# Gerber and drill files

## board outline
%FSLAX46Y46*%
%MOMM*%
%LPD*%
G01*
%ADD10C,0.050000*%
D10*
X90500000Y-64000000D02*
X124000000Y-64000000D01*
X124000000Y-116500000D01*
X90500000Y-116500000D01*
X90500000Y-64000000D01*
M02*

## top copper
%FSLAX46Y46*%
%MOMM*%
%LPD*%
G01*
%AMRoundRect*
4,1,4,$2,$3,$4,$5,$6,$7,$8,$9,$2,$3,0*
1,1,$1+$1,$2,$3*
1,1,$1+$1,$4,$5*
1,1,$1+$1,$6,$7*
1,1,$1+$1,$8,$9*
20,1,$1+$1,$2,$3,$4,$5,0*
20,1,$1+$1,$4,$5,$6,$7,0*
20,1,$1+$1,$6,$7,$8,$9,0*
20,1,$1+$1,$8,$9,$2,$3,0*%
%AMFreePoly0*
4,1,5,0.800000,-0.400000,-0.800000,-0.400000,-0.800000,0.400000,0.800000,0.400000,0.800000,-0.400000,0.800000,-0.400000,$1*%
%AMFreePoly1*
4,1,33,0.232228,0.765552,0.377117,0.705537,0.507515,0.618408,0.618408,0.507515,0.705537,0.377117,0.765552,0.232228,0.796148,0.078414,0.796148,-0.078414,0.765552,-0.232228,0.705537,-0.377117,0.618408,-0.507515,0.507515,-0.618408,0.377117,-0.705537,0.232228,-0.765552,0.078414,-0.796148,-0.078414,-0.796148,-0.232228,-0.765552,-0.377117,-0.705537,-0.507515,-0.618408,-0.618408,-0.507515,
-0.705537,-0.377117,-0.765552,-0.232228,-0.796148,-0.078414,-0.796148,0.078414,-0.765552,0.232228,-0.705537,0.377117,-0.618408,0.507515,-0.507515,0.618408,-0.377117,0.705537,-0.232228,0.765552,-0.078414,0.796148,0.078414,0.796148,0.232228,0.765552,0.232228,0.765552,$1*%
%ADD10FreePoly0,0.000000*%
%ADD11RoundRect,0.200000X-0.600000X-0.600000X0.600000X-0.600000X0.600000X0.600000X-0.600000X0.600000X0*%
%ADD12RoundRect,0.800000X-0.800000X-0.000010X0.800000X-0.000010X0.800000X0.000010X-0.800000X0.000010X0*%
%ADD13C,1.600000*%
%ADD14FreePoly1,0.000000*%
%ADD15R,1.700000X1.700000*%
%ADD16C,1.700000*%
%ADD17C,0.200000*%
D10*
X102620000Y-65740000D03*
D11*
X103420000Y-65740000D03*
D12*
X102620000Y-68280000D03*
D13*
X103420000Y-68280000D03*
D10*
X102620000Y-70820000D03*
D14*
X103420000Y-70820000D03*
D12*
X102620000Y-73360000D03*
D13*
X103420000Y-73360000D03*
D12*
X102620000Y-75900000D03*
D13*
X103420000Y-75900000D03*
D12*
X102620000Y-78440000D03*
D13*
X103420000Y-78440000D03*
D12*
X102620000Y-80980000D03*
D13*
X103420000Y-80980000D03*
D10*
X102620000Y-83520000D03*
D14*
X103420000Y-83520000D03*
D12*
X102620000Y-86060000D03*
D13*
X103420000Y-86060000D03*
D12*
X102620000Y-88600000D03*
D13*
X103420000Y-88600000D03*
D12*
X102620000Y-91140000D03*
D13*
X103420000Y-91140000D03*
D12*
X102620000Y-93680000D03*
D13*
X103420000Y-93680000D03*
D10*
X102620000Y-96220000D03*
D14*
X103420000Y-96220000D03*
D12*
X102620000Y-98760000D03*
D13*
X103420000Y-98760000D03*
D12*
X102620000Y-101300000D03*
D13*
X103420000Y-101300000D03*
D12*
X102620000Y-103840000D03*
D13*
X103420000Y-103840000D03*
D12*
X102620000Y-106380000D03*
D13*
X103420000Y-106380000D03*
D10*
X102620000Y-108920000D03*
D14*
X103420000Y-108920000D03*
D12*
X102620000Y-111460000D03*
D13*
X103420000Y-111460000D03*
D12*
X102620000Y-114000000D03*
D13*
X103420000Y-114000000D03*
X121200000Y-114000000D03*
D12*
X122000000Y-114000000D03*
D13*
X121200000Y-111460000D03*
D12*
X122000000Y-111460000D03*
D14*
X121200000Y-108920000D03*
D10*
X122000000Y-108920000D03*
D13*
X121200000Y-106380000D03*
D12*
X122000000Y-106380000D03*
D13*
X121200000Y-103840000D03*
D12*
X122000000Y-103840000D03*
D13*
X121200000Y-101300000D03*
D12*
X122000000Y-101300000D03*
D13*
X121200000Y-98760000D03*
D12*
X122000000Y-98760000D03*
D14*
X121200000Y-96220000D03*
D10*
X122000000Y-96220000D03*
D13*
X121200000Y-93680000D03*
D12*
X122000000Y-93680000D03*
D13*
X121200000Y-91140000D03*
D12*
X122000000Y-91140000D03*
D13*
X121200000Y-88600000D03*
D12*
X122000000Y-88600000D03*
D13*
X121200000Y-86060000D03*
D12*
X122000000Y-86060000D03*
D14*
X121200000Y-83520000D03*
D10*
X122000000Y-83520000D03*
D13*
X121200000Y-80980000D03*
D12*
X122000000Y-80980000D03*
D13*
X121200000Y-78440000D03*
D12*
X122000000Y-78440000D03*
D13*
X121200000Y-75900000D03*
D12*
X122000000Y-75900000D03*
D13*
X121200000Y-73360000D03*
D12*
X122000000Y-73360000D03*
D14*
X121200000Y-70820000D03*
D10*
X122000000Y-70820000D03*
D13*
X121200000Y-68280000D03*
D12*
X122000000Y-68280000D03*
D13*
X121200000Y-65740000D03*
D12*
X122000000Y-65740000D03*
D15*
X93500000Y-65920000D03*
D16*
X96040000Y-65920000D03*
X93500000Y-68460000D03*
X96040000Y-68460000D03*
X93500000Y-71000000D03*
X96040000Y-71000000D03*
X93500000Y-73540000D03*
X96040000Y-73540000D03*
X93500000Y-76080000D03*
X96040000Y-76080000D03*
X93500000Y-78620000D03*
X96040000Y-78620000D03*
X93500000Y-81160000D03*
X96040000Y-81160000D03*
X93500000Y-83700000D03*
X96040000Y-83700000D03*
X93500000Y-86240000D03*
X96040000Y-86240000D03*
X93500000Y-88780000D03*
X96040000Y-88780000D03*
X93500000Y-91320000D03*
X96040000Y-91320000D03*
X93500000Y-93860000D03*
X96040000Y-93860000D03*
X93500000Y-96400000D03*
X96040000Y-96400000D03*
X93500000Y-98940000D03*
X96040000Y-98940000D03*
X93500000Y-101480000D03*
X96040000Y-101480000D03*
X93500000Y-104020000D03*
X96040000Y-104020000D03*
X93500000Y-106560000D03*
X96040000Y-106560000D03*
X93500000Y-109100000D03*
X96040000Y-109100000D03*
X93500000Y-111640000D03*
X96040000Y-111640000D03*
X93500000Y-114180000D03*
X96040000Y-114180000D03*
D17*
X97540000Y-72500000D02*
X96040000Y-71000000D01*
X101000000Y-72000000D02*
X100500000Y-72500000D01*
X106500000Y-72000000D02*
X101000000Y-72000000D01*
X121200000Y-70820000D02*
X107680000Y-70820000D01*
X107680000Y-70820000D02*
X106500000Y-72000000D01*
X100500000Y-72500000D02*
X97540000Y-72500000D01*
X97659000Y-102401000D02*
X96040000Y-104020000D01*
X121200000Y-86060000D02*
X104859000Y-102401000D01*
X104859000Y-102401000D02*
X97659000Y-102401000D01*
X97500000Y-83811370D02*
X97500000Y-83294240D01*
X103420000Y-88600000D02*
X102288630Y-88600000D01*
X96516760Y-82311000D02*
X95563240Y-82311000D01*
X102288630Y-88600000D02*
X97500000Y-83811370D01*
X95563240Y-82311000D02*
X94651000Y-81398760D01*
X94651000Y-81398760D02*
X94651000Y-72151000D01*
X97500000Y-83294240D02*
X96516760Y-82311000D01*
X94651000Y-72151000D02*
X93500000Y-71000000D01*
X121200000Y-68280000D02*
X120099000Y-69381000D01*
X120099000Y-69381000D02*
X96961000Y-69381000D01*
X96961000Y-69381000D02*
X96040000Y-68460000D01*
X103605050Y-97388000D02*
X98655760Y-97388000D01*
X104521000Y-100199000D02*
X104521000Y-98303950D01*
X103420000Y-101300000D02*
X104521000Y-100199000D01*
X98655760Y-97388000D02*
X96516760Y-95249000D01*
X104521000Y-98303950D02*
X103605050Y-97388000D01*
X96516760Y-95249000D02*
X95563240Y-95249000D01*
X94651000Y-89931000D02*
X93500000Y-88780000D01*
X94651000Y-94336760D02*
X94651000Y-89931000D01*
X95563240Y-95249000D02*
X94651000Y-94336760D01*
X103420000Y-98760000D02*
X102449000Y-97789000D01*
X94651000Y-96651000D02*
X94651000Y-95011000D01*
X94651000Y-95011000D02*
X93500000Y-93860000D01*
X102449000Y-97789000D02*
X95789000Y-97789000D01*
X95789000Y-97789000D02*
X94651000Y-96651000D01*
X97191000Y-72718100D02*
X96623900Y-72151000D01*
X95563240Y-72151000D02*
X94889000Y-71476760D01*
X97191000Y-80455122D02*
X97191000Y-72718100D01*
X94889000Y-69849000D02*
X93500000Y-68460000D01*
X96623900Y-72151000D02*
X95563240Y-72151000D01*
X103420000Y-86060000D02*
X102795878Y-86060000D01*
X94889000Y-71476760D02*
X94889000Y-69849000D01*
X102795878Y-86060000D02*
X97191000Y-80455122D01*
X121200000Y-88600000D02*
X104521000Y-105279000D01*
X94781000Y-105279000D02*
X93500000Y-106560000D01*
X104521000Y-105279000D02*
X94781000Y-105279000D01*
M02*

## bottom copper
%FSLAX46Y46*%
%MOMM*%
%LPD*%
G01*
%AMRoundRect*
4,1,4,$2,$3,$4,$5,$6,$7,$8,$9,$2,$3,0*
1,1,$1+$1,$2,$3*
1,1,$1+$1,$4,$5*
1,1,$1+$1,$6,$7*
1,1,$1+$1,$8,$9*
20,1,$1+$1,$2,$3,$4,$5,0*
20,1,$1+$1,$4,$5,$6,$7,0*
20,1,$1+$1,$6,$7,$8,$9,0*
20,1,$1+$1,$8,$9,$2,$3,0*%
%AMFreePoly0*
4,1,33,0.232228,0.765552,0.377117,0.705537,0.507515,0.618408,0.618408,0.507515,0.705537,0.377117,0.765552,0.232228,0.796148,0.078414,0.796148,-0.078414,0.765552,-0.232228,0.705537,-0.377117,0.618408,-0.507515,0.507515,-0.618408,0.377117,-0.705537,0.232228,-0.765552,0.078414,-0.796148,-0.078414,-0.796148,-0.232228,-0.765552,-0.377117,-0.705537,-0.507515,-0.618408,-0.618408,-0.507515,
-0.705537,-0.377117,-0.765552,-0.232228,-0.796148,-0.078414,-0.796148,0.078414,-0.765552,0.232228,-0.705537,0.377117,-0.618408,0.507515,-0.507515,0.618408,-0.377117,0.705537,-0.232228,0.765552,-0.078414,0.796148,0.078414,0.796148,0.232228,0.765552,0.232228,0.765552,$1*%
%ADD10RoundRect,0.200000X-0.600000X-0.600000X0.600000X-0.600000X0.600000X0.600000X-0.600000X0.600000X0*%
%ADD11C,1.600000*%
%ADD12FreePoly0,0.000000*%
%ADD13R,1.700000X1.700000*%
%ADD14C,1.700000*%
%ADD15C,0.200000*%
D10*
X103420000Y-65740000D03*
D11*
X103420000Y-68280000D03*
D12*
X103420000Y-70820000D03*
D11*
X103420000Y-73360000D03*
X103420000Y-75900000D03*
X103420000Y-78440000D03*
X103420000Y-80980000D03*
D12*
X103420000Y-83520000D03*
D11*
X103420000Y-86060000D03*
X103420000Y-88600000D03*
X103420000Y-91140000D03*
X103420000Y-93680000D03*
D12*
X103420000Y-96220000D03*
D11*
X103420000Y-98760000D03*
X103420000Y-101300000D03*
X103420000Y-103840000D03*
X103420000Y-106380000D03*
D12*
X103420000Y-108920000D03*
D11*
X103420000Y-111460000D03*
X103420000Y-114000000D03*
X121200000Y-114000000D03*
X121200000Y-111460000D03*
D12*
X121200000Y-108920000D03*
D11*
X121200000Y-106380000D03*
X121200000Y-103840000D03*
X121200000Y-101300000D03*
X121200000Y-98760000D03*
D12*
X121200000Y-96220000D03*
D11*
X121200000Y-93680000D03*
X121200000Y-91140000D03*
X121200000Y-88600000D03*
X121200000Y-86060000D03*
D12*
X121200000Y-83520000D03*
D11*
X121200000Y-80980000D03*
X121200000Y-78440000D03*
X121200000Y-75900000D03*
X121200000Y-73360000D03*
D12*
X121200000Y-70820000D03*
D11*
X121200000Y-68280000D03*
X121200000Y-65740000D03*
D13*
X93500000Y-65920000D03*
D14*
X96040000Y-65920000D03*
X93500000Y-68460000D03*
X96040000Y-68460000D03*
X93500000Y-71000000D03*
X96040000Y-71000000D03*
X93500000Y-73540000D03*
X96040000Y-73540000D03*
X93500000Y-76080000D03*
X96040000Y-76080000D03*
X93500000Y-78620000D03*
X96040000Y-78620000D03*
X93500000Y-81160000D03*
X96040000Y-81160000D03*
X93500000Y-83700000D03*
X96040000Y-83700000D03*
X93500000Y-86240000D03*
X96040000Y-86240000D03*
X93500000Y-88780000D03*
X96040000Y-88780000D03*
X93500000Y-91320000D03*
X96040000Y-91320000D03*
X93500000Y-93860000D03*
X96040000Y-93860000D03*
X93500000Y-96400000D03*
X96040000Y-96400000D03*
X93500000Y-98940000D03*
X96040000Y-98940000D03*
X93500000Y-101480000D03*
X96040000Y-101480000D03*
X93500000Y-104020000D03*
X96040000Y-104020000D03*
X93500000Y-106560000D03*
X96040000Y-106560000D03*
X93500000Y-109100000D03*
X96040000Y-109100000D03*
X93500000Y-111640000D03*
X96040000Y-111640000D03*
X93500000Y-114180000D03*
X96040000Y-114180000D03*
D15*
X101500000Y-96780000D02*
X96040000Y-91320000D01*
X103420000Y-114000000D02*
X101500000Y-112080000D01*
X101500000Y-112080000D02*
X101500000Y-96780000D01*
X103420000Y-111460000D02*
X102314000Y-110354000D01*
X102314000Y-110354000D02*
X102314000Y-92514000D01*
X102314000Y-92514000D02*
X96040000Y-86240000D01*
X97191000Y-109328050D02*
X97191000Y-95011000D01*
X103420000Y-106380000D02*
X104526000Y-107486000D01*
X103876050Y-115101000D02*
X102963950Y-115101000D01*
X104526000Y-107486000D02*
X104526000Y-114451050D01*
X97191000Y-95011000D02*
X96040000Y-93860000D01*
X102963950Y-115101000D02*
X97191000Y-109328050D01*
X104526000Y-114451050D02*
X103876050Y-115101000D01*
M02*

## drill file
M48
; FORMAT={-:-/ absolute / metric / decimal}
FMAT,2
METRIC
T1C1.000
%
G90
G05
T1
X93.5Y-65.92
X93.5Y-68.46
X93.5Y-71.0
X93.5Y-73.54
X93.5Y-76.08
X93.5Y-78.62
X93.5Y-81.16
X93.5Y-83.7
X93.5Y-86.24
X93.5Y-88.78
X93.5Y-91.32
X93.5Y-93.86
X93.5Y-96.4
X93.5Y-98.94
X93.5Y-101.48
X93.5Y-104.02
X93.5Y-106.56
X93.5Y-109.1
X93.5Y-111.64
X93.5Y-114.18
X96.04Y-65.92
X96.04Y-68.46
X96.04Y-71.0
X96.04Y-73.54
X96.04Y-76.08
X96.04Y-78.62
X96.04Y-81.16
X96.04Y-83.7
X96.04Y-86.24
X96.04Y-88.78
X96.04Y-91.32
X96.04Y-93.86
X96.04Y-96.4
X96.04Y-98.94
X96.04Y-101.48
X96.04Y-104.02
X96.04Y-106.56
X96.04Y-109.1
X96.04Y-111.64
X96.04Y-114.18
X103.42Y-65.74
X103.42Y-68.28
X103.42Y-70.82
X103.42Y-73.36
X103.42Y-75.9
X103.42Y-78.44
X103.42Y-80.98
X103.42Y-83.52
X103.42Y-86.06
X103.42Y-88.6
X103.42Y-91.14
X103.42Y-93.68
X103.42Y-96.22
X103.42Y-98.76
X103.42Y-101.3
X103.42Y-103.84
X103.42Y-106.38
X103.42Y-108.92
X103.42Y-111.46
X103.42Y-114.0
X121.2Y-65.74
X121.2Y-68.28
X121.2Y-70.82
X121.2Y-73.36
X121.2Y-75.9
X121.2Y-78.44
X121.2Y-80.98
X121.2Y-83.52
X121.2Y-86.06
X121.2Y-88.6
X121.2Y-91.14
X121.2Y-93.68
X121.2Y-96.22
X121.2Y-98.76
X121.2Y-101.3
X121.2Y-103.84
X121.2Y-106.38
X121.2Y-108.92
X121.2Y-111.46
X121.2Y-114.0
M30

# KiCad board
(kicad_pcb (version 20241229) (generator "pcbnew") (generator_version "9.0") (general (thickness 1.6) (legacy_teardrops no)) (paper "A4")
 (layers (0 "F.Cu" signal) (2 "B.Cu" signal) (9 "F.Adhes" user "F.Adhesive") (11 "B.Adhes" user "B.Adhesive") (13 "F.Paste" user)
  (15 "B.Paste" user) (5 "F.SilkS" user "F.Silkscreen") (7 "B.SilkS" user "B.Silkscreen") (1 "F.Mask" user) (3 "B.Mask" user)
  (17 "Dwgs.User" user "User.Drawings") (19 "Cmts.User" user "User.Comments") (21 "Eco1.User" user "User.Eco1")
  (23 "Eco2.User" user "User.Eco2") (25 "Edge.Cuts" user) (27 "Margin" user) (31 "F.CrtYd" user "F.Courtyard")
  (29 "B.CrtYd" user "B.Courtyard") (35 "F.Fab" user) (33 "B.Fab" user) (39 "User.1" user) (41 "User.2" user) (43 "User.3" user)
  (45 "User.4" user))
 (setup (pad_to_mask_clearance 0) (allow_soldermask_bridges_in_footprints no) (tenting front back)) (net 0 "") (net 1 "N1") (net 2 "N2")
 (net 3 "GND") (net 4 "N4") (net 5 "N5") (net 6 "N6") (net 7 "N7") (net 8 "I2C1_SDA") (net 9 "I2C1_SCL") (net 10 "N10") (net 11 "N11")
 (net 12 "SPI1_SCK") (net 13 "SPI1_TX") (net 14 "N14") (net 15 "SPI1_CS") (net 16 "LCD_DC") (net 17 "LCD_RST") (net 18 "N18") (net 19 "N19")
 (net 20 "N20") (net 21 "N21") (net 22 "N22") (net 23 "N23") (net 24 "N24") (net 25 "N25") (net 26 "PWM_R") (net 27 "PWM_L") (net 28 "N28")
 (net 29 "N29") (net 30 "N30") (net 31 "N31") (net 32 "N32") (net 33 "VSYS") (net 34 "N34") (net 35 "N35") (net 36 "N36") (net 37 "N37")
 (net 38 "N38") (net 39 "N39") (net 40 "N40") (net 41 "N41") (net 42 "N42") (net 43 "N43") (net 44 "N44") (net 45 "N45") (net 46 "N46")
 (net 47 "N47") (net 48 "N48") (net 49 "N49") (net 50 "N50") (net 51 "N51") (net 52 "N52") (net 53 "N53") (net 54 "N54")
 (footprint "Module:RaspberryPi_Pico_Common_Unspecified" (layer "F.Cu") (at 112.31 89.87)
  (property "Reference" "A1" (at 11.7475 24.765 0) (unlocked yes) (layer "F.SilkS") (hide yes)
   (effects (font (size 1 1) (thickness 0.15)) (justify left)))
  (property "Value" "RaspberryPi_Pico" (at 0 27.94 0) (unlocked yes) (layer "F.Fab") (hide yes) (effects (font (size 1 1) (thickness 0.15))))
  (pad "1" smd custom (at -9.69 -24.13) (size 1.6 0.8) (layers "F.Cu" "F.Mask") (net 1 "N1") (options (clearance outline) (anchor rect))
   (primitives))
  (pad "1" thru_hole roundrect (at -8.89 -24.13) (size 1.6 1.6) (drill 1) (layers "*.Cu" "*.Mask") (remove_unused_layers no)
   (roundrect_rratio 0.125) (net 1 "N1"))
  (pad "2" smd roundrect (at -9.69 -21.59) (size 3.2 1.6) (layers "F.Cu" "F.Mask") (roundrect_rratio 0.5) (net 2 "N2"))
  (pad "2" thru_hole circle (at -8.89 -21.59) (size 1.6 1.6) (drill 1) (layers "*.Cu" "*.Mask") (remove_unused_layers no) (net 2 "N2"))
  (pad "3" smd custom (at -9.69 -19.05) (size 1.6 0.8) (layers "F.Cu" "F.Mask") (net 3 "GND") (options (clearance outline) (anchor rect))
   (primitives))
  (pad "3" thru_hole custom (at -8.89 -19.05) (size 1.6 1.6) (drill 1) (layers "*.Cu" "*.Mask") (remove_unused_layers no) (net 3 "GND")
   (options (clearance outline) (anchor circle)) (primitives))
  (pad "4" smd roundrect (at -9.69 -16.51) (size 3.2 1.6) (layers "F.Cu" "F.Mask") (roundrect_rratio 0.5) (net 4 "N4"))
  (pad "4" thru_hole circle (at -8.89 -16.51) (size 1.6 1.6) (drill 1) (layers "*.Cu" "*.Mask") (remove_unused_layers no) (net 4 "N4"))
  (pad "5" smd roundrect (at -9.69 -13.97) (size 3.2 1.6) (layers "F.Cu" "F.Mask") (roundrect_rratio 0.5) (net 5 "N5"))
  (pad "5" thru_hole circle (at -8.89 -13.97) (size 1.6 1.6) (drill 1) (layers "*.Cu" "*.Mask") (remove_unused_layers no) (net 5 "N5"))
  (pad "6" smd roundrect (at -9.69 -11.43) (size 3.2 1.6) (layers "F.Cu" "F.Mask") (roundrect_rratio 0.5) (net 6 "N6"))
  (pad "6" thru_hole circle (at -8.89 -11.43) (size 1.6 1.6) (drill 1) (layers "*.Cu" "*.Mask") (remove_unused_layers no) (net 6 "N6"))
  (pad "7" smd roundrect (at -9.69 -8.89) (size 3.2 1.6) (layers "F.Cu" "F.Mask") (roundrect_rratio 0.5) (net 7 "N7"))
  (pad "7" thru_hole circle (at -8.89 -8.89) (size 1.6 1.6) (drill 1) (layers "*.Cu" "*.Mask") (remove_unused_layers no) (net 7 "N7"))
  (pad "8" smd custom (at -9.69 -6.35) (size 1.6 0.8) (layers "F.Cu" "F.Mask") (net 3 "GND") (options (clearance outline) (anchor rect))
   (primitives))
  (pad "8" thru_hole custom (at -8.89 -6.35) (size 1.6 1.6) (drill 1) (layers "*.Cu" "*.Mask") (remove_unused_layers no) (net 3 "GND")
   (options (clearance outline) (anchor circle)) (primitives))
  (pad "9" smd roundrect (at -9.69 -3.81) (size 3.2 1.6) (layers "F.Cu" "F.Mask") (roundrect_rratio 0.5) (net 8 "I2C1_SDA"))
  (pad "9" thru_hole circle (at -8.89 -3.81) (size 1.6 1.6) (drill 1) (layers "*.Cu" "*.Mask") (remove_unused_layers no) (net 8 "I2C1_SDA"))
  (pad "10" smd roundrect (at -9.69 -1.27) (size 3.2 1.6) (layers "F.Cu" "F.Mask") (roundrect_rratio 0.5) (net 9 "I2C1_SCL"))
  (pad "10" thru_hole circle (at -8.89 -1.27) (size 1.6 1.6) (drill 1) (layers "*.Cu" "*.Mask") (remove_unused_layers no) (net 9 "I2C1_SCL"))
  (pad "11" smd roundrect (at -9.69 1.27) (size 3.2 1.6) (layers "F.Cu" "F.Mask") (roundrect_rratio 0.5) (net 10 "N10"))
  (pad "11" thru_hole circle (at -8.89 1.27) (size 1.6 1.6) (drill 1) (layers "*.Cu" "*.Mask") (remove_unused_layers no) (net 10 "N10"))
  (pad "12" smd roundrect (at -9.69 3.81) (size 3.2 1.6) (layers "F.Cu" "F.Mask") (roundrect_rratio 0.5) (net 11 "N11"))
  (pad "12" thru_hole circle (at -8.89 3.81) (size 1.6 1.6) (drill 1) (layers "*.Cu" "*.Mask") (remove_unused_layers no) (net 11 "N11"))
  (pad "13" smd custom (at -9.69 6.35) (size 1.6 0.8) (layers "F.Cu" "F.Mask") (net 3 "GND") (options (clearance outline) (anchor rect))
   (primitives))
  (pad "13" thru_hole custom (at -8.89 6.35) (size 1.6 1.6) (drill 1) (layers "*.Cu" "*.Mask") (remove_unused_layers no) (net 3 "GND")
   (options (clearance outline) (anchor circle)) (primitives))
  (pad "14" smd roundrect (at -9.69 8.89) (size 3.2 1.6) (layers "F.Cu" "F.Mask") (roundrect_rratio 0.5) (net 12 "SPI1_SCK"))
  (pad "14" thru_hole circle (at -8.89 8.89) (size 1.6 1.6) (drill 1) (layers "*.Cu" "*.Mask") (remove_unused_layers no) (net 12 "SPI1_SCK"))
  (pad "15" smd roundrect (at -9.69 11.43) (size 3.2 1.6) (layers "F.Cu" "F.Mask") (roundrect_rratio 0.5) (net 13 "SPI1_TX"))
  (pad "15" thru_hole circle (at -8.89 11.43) (size 1.6 1.6) (drill 1) (layers "*.Cu" "*.Mask") (remove_unused_layers no) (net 13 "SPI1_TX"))
  (pad "16" smd roundrect (at -9.69 13.97) (size 3.2 1.6) (layers "F.Cu" "F.Mask") (roundrect_rratio 0.5) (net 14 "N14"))
  (pad "16" thru_hole circle (at -8.89 13.97) (size 1.6 1.6) (drill 1) (layers "*.Cu" "*.Mask") (remove_unused_layers no) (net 14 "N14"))
  (pad "17" smd roundrect (at -9.69 16.51) (size 3.2 1.6) (layers "F.Cu" "F.Mask") (roundrect_rratio 0.5) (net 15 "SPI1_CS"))
  (pad "17" thru_hole circle (at -8.89 16.51) (size 1.6 1.6) (drill 1) (layers "*.Cu" "*.Mask") (remove_unused_layers no) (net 15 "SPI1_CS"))
  (pad "18" smd custom (at -9.69 19.05) (size 1.6 0.8) (layers "F.Cu" "F.Mask") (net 3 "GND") (options (clearance outline) (anchor rect))
   (primitives))
  (pad "18" thru_hole custom (at -8.89 19.05) (size 1.6 1.6) (drill 1) (layers "*.Cu" "*.Mask") (remove_unused_layers no) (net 3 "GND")
   (options (clearance outline) (anchor circle)) (primitives))
  (pad "19" smd roundrect (at -9.69 21.59) (size 3.2 1.6) (layers "F.Cu" "F.Mask") (roundrect_rratio 0.5) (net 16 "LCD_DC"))
  (pad "19" thru_hole circle (at -8.89 21.59) (size 1.6 1.6) (drill 1) (layers "*.Cu" "*.Mask") (remove_unused_layers no) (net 16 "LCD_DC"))
  (pad "20" smd roundrect (at -9.69 24.13) (size 3.2 1.6) (layers "F.Cu" "F.Mask") (roundrect_rratio 0.5) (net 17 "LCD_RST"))
  (pad "20" thru_hole circle (at -8.89 24.13) (size 1.6 1.6) (drill 1) (layers "*.Cu" "*.Mask") (remove_unused_layers no) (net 17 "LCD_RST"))
  (pad "21" thru_hole circle (at 8.89 24.13) (size 1.6 1.6) (drill 1) (layers "*.Cu" "*.Mask") (remove_unused_layers no) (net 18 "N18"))
  (pad "21" smd roundrect (at 9.69 24.13) (size 3.2 1.6) (layers "F.Cu" "F.Mask") (roundrect_rratio 0.5) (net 18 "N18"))
  (pad "22" thru_hole circle (at 8.89 21.59) (size 1.6 1.6) (drill 1) (layers "*.Cu" "*.Mask") (remove_unused_layers no) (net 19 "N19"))
  (pad "22" smd roundrect (at 9.69 21.59) (size 3.2 1.6) (layers "F.Cu" "F.Mask") (roundrect_rratio 0.5) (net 19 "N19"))
  (pad "23" thru_hole custom (at 8.89 19.05) (size 1.6 1.6) (drill 1) (layers "*.Cu" "*.Mask") (remove_unused_layers no) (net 3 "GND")
   (options (clearance outline) (anchor circle)) (primitives))
  (pad "23" smd custom (at 9.69 19.05) (size 1.6 0.8) (layers "F.Cu" "F.Mask") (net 3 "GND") (options (clearance outline) (anchor rect))
   (primitives))
  (pad "24" thru_hole circle (at 8.89 16.51) (size 1.6 1.6) (drill 1) (layers "*.Cu" "*.Mask") (remove_unused_layers no) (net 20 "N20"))
  (pad "24" smd roundrect (at 9.69 16.51) (size 3.2 1.6) (layers "F.Cu" "F.Mask") (roundrect_rratio 0.5) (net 20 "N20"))
  (pad "25" thru_hole circle (at 8.89 13.97) (size 1.6 1.6) (drill 1) (layers "*.Cu" "*.Mask") (remove_unused_layers no) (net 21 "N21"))
  (pad "25" smd roundrect (at 9.69 13.97) (size 3.2 1.6) (layers "F.Cu" "F.Mask") (roundrect_rratio 0.5) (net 21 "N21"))
  (pad "26" thru_hole circle (at 8.89 11.43) (size 1.6 1.6) (drill 1) (layers "*.Cu" "*.Mask") (remove_unused_layers no) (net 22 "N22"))
  (pad "26" smd roundrect (at 9.69 11.43) (size 3.2 1.6) (layers "F.Cu" "F.Mask") (roundrect_rratio 0.5) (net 22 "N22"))
  (pad "27" thru_hole circle (at 8.89 8.89) (size 1.6 1.6) (drill 1) (layers "*.Cu" "*.Mask") (remove_unused_layers no) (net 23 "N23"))
  (pad "27" smd roundrect (at 9.69 8.89) (size 3.2 1.6) (layers "F.Cu" "F.Mask") (roundrect_rratio 0.5) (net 23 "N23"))
  (pad "28" thru_hole custom (at 8.89 6.35) (size 1.6 1.6) (drill 1) (layers "*.Cu" "*.Mask") (remove_unused_layers no) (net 3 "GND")
   (options (clearance outline) (anchor circle)) (primitives))
  (pad "28" smd custom (at 9.69 6.35) (size 1.6 0.8) (layers "F.Cu" "F.Mask") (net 3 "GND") (options (clearance outline) (anchor rect))
   (primitives))
  (pad "29" thru_hole circle (at 8.89 3.81) (size 1.6 1.6) (drill 1) (layers "*.Cu" "*.Mask") (remove_unused_layers no) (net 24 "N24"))
  (pad "29" smd roundrect (at 9.69 3.81) (size 3.2 1.6) (layers "F.Cu" "F.Mask") (roundrect_rratio 0.5) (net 24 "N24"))
  (pad "30" thru_hole circle (at 8.89 1.27) (size 1.6 1.6) (drill 1) (layers "*.Cu" "*.Mask") (remove_unused_layers no) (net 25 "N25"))
  (pad "30" smd roundrect (at 9.69 1.27) (size 3.2 1.6) (layers "F.Cu" "F.Mask") (roundrect_rratio 0.5) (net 25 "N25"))
  (pad "31" thru_hole circle (at 8.89 -1.27) (size 1.6 1.6) (drill 1) (layers "*.Cu" "*.Mask") (remove_unused_layers no) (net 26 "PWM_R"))
  (pad "31" smd roundrect (at 9.69 -1.27) (size 3.2 1.6) (layers "F.Cu" "F.Mask") (roundrect_rratio 0.5) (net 26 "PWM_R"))
  (pad "32" thru_hole circle (at 8.89 -3.81) (size 1.6 1.6) (drill 1) (layers "*.Cu" "*.Mask") (remove_unused_layers no) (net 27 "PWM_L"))
  (pad "32" smd roundrect (at 9.69 -3.81) (size 3.2 1.6) (layers "F.Cu" "F.Mask") (roundrect_rratio 0.5) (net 27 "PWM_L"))
  (pad "33" thru_hole custom (at 8.89 -6.35) (size 1.6 1.6) (drill 1) (layers "*.Cu" "*.Mask") (remove_unused_layers no) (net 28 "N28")
   (options (clearance outline) (anchor circle)) (primitives))
  (pad "33" smd custom (at 9.69 -6.35) (size 1.6 0.8) (layers "F.Cu" "F.Mask") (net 28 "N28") (options (clearance outline) (anchor rect))
   (primitives))
  (pad "34" thru_hole circle (at 8.89 -8.89) (size 1.6 1.6) (drill 1) (layers "*.Cu" "*.Mask") (remove_unused_layers no) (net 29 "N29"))
  (pad "34" smd roundrect (at 9.69 -8.89) (size 3.2 1.6) (layers "F.Cu" "F.Mask") (roundrect_rratio 0.5) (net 29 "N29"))
  (pad "35" thru_hole circle (at 8.89 -11.43) (size 1.6 1.6) (drill 1) (layers "*.Cu" "*.Mask") (remove_unused_layers no) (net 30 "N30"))
  (pad "35" smd roundrect (at 9.69 -11.43) (size 3.2 1.6) (layers "F.Cu" "F.Mask") (roundrect_rratio 0.5) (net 30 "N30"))
  (pad "36" thru_hole circle (at 8.89 -13.97) (size 1.6 1.6) (drill 1) (layers "*.Cu" "*.Mask") (remove_unused_layers no) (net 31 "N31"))
  (pad "36" smd roundrect (at 9.69 -13.97) (size 3.2 1.6) (layers "F.Cu" "F.Mask") (roundrect_rratio 0.5) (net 31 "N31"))
  (pad "37" thru_hole circle (at 8.89 -16.51) (size 1.6 1.6) (drill 1) (layers "*.Cu" "*.Mask") (remove_unused_layers no) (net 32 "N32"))
  (pad "37" smd roundrect (at 9.69 -16.51) (size 3.2 1.6) (layers "F.Cu" "F.Mask") (roundrect_rratio 0.5) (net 32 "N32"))
  (pad "38" thru_hole custom (at 8.89 -19.05) (size 1.6 1.6) (drill 1) (layers "*.Cu" "*.Mask") (remove_unused_layers no) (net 3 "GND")
   (options (clearance outline) (anchor circle)) (primitives))
  (pad "38" smd custom (at 9.69 -19.05) (size 1.6 0.8) (layers "F.Cu" "F.Mask") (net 3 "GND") (options (clearance outline) (anchor rect))
   (primitives))
  (pad "39" thru_hole circle (at 8.89 -21.59) (size 1.6 1.6) (drill 1) (layers "*.Cu" "*.Mask") (remove_unused_layers no) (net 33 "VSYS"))
  (pad "39" smd roundrect (at 9.69 -21.59) (size 3.2 1.6) (layers "F.Cu" "F.Mask") (roundrect_rratio 0.5) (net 33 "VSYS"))
  (pad "40" thru_hole circle (at 8.89 -24.13) (size 1.6 1.6) (drill 1) (layers "*.Cu" "*.Mask") (remove_unused_layers no) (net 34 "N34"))
  (pad "40" smd roundrect (at 9.69 -24.13) (size 3.2 1.6) (layers "F.Cu" "F.Mask") (roundrect_rratio 0.5) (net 34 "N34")))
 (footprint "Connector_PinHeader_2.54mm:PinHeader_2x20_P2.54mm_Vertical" (layer "F.Cu") (at 93.5 65.92)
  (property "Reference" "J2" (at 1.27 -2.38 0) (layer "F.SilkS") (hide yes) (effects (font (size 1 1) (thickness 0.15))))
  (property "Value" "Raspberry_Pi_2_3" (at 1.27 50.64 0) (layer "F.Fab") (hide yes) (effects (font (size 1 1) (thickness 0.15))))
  (pad "1" thru_hole rect (at 0 0) (size 1.7 1.7) (drill 1) (layers "*.Cu" "*.Mask") (remove_unused_layers no) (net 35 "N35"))
  (pad "2" thru_hole circle (at 2.54 0) (size 1.7 1.7) (drill 1) (layers "*.Cu" "*.Mask") (remove_unused_layers no) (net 33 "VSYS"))
  (pad "3" thru_hole circle (at 0 2.54) (size 1.7 1.7) (drill 1) (layers "*.Cu" "*.Mask") (remove_unused_layers no) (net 8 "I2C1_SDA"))
  (pad "4" thru_hole circle (at 2.54 2.54) (size 1.7 1.7) (drill 1) (layers "*.Cu" "*.Mask") (remove_unused_layers no) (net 33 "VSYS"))
  (pad "5" thru_hole circle (at 0 5.08) (size 1.7 1.7) (drill 1) (layers "*.Cu" "*.Mask") (remove_unused_layers no) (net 9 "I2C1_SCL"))
  (pad "6" thru_hole circle (at 2.54 5.08) (size 1.7 1.7) (drill 1) (layers "*.Cu" "*.Mask") (remove_unused_layers no) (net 3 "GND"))
  (pad "7" thru_hole circle (at 0 7.62) (size 1.7 1.7) (drill 1) (layers "*.Cu" "*.Mask") (remove_unused_layers no) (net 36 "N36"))
  (pad "8" thru_hole circle (at 2.54 7.62) (size 1.7 1.7) (drill 1) (layers "*.Cu" "*.Mask") (remove_unused_layers no) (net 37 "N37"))
  (pad "9" thru_hole circle (at 0 10.16) (size 1.7 1.7) (drill 1) (layers "*.Cu" "*.Mask") (remove_unused_layers no) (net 3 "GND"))
  (pad "10" thru_hole circle (at 2.54 10.16) (size 1.7 1.7) (drill 1) (layers "*.Cu" "*.Mask") (remove_unused_layers no) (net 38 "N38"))
  (pad "11" thru_hole circle (at 0 12.7) (size 1.7 1.7) (drill 1) (layers "*.Cu" "*.Mask") (remove_unused_layers no) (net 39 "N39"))
  (pad "12" thru_hole circle (at 2.54 12.7) (size 1.7 1.7) (drill 1) (layers "*.Cu" "*.Mask") (remove_unused_layers no) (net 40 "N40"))
  (pad "13" thru_hole circle (at 0 15.24) (size 1.7 1.7) (drill 1) (layers "*.Cu" "*.Mask") (remove_unused_layers no) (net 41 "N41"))
  (pad "14" thru_hole circle (at 2.54 15.24) (size 1.7 1.7) (drill 1) (layers "*.Cu" "*.Mask") (remove_unused_layers no) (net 3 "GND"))
  (pad "15" thru_hole circle (at 0 17.78) (size 1.7 1.7) (drill 1) (layers "*.Cu" "*.Mask") (remove_unused_layers no) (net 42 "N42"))
  (pad "16" thru_hole circle (at 2.54 17.78) (size 1.7 1.7) (drill 1) (layers "*.Cu" "*.Mask") (remove_unused_layers no) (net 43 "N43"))
  (pad "17" thru_hole circle (at 0 20.32) (size 1.7 1.7) (drill 1) (layers "*.Cu" "*.Mask") (remove_unused_layers no) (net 35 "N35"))
  (pad "18" thru_hole circle (at 2.54 20.32) (size 1.7 1.7) (drill 1) (layers "*.Cu" "*.Mask") (remove_unused_layers no) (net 16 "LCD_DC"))
  (pad "19" thru_hole circle (at 0 22.86) (size 1.7 1.7) (drill 1) (layers "*.Cu" "*.Mask") (remove_unused_layers no) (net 13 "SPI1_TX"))
  (pad "20" thru_hole circle (at 2.54 22.86) (size 1.7 1.7) (drill 1) (layers "*.Cu" "*.Mask") (remove_unused_layers no) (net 3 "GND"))
  (pad "21" thru_hole circle (at 0 25.4) (size 1.7 1.7) (drill 1) (layers "*.Cu" "*.Mask") (remove_unused_layers no) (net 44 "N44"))
  (pad "22" thru_hole circle (at 2.54 25.4) (size 1.7 1.7) (drill 1) (layers "*.Cu" "*.Mask") (remove_unused_layers no) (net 17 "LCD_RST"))
  (pad "23" thru_hole circle (at 0 27.94) (size 1.7 1.7) (drill 1) (layers "*.Cu" "*.Mask") (remove_unused_layers no) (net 12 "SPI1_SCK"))
  (pad "24" thru_hole circle (at 2.54 27.94) (size 1.7 1.7) (drill 1) (layers "*.Cu" "*.Mask") (remove_unused_layers no) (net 15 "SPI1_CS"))
  (pad "25" thru_hole circle (at 0 30.48) (size 1.7 1.7) (drill 1) (layers "*.Cu" "*.Mask") (remove_unused_layers no) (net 3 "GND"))
  (pad "26" thru_hole circle (at 2.54 30.48) (size 1.7 1.7) (drill 1) (layers "*.Cu" "*.Mask") (remove_unused_layers no) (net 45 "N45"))
  (pad "27" thru_hole circle (at 0 33.02) (size 1.7 1.7) (drill 1) (layers "*.Cu" "*.Mask") (remove_unused_layers no) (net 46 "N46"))
  (pad "28" thru_hole circle (at 2.54 33.02) (size 1.7 1.7) (drill 1) (layers "*.Cu" "*.Mask") (remove_unused_layers no) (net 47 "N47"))
  (pad "29" thru_hole circle (at 0 35.56) (size 1.7 1.7) (drill 1) (layers "*.Cu" "*.Mask") (remove_unused_layers no) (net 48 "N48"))
  (pad "30" thru_hole circle (at 2.54 35.56) (size 1.7 1.7) (drill 1) (layers "*.Cu" "*.Mask") (remove_unused_layers no) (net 3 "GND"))
  (pad "31" thru_hole circle (at 0 38.1) (size 1.7 1.7) (drill 1) (layers "*.Cu" "*.Mask") (remove_unused_layers no) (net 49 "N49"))
  (pad "32" thru_hole circle (at 2.54 38.1) (size 1.7 1.7) (drill 1) (layers "*.Cu" "*.Mask") (remove_unused_layers no) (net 27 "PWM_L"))
  (pad "33" thru_hole circle (at 0 40.64) (size 1.7 1.7) (drill 1) (layers "*.Cu" "*.Mask") (remove_unused_layers no) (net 26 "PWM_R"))
  (pad "34" thru_hole circle (at 2.54 40.64) (size 1.7 1.7) (drill 1) (layers "*.Cu" "*.Mask") (remove_unused_layers no) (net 3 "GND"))
  (pad "35" thru_hole circle (at 0 43.18) (size 1.7 1.7) (drill 1) (layers "*.Cu" "*.Mask") (remove_unused_layers no) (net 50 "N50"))
  (pad "36" thru_hole circle (at 2.54 43.18) (size 1.7 1.7) (drill 1) (layers "*.Cu" "*.Mask") (remove_unused_layers no) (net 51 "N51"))
  (pad "37" thru_hole circle (at 0 45.72) (size 1.7 1.7) (drill 1) (layers "*.Cu" "*.Mask") (remove_unused_layers no) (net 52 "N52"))
  (pad "38" thru_hole circle (at 2.54 45.72) (size 1.7 1.7) (drill 1) (layers "*.Cu" "*.Mask") (remove_unused_layers no) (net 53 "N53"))
  (pad "39" thru_hole circle (at 0 48.26) (size 1.7 1.7) (drill 1) (layers "*.Cu" "*.Mask") (remove_unused_layers no) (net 3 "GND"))
  (pad "40" thru_hole circle (at 2.54 48.26) (size 1.7 1.7) (drill 1) (layers "*.Cu" "*.Mask") (remove_unused_layers no) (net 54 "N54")))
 (gr_rect (start 90.5 64) (end 124 116.5) (stroke (width 0.05) (type default)) (fill no) (layer "Edge.Cuts"))
 (segment (start 97.54 72.5) (end 96.04 71) (width 0.2) (layer "F.Cu") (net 3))
 (segment (start 101 72) (end 100.5 72.5) (width 0.2) (layer "F.Cu") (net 3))
 (segment (start 106.5 72) (end 101 72) (width 0.2) (layer "F.Cu") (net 3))
 (segment (start 121.2 70.82) (end 107.68 70.82) (width 0.2) (layer "F.Cu") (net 3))
 (segment (start 107.68 70.82) (end 106.5 72) (width 0.2) (layer "F.Cu") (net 3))
 (segment (start 100.5 72.5) (end 97.54 72.5) (width 0.2) (layer "F.Cu") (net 3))
 (segment (start 97.659 102.401) (end 96.04 104.02) (width 0.2) (layer "F.Cu") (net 27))
 (segment (start 121.2 86.06) (end 104.859 102.401) (width 0.2) (layer "F.Cu") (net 27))
 (segment (start 104.859 102.401) (end 97.659 102.401) (width 0.2) (layer "F.Cu") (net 27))
 (segment (start 101.5 96.78) (end 96.04 91.32) (width 0.2) (layer "B.Cu") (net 17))
 (segment (start 103.42 114) (end 101.5 112.08) (width 0.2) (layer "B.Cu") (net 17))
 (segment (start 101.5 112.08) (end 101.5 96.78) (width 0.2) (layer "B.Cu") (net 17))
 (segment (start 97.5 83.81137) (end 97.5 83.29424) (width 0.2) (layer "F.Cu") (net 9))
 (segment (start 103.42 88.6) (end 102.28863 88.6) (width 0.2) (layer "F.Cu") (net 9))
 (segment (start 96.51676 82.311) (end 95.56324 82.311) (width 0.2) (layer "F.Cu") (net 9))
 (segment (start 102.28863 88.6) (end 97.5 83.81137) (width 0.2) (layer "F.Cu") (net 9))
 (segment (start 95.56324 82.311) (end 94.651 81.39876) (width 0.2) (layer "F.Cu") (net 9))
 (segment (start 94.651 81.39876) (end 94.651 72.151) (width 0.2) (layer "F.Cu") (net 9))
 (segment (start 97.5 83.29424) (end 96.51676 82.311) (width 0.2) (layer "F.Cu") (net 9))
 (segment (start 94.651 72.151) (end 93.5 71) (width 0.2) (layer "F.Cu") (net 9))
 (segment (start 121.2 68.28) (end 120.099 69.381) (width 0.2) (layer "F.Cu") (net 33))
 (segment (start 120.099 69.381) (end 96.961 69.381) (width 0.2) (layer "F.Cu") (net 33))
 (segment (start 96.961 69.381) (end 96.04 68.46) (width 0.2) (layer "F.Cu") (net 33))
 (segment (start 103.60505 97.388) (end 98.65576 97.388) (width 0.2) (layer "F.Cu") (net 13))
 (segment (start 104.521 100.199) (end 104.521 98.30395) (width 0.2) (layer "F.Cu") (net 13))
 (segment (start 103.42 101.3) (end 104.521 100.199) (width 0.2) (layer "F.Cu") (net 13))
 (segment (start 98.65576 97.388) (end 96.51676 95.249) (width 0.2) (layer "F.Cu") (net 13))
 (segment (start 104.521 98.30395) (end 103.60505 97.388) (width 0.2) (layer "F.Cu") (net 13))
 (segment (start 96.51676 95.249) (end 95.56324 95.249) (width 0.2) (layer "F.Cu") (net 13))
 (segment (start 94.651 89.931) (end 93.5 88.78) (width 0.2) (layer "F.Cu") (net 13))
 (segment (start 94.651 94.33676) (end 94.651 89.931) (width 0.2) (layer "F.Cu") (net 13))
 (segment (start 95.56324 95.249) (end 94.651 94.33676) (width 0.2) (layer "F.Cu") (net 13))
 (segment (start 103.42 98.76) (end 102.449 97.789) (width 0.2) (layer "F.Cu") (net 12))
 (segment (start 94.651 96.651) (end 94.651 95.011) (width 0.2) (layer "F.Cu") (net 12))
 (segment (start 94.651 95.011) (end 93.5 93.86) (width 0.2) (layer "F.Cu") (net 12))
 (segment (start 102.449 97.789) (end 95.789 97.789) (width 0.2) (layer "F.Cu") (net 12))
 (segment (start 95.789 97.789) (end 94.651 96.651) (width 0.2) (layer "F.Cu") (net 12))
 (segment (start 103.42 111.46) (end 102.314 110.354) (width 0.2) (layer "B.Cu") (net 16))
 (segment (start 102.314 110.354) (end 102.314 92.514) (width 0.2) (layer "B.Cu") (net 16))
 (segment (start 102.314 92.514) (end 96.04 86.24) (width 0.2) (layer "B.Cu") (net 16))
 (segment (start 97.191 72.7181) (end 96.6239 72.151) (width 0.2) (layer "F.Cu") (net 8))
 (segment (start 95.56324 72.151) (end 94.889 71.47676) (width 0.2) (layer "F.Cu") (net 8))
 (segment (start 97.191 80.455122) (end 97.191 72.7181) (width 0.2) (layer "F.Cu") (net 8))
 (segment (start 94.889 69.849) (end 93.5 68.46) (width 0.2) (layer "F.Cu") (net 8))
 (segment (start 96.6239 72.151) (end 95.56324 72.151) (width 0.2) (layer "F.Cu") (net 8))
 (segment (start 103.42 86.06) (end 102.795878 86.06) (width 0.2) (layer "F.Cu") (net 8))
 (segment (start 94.889 71.47676) (end 94.889 69.849) (width 0.2) (layer "F.Cu") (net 8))
 (segment (start 102.795878 86.06) (end 97.191 80.455122) (width 0.2) (layer "F.Cu") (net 8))
 (segment (start 97.191 109.32805) (end 97.191 95.011) (width 0.2) (layer "B.Cu") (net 15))
 (segment (start 103.42 106.38) (end 104.526 107.486) (width 0.2) (layer "B.Cu") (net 15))
 (segment (start 103.87605 115.101) (end 102.96395 115.101) (width 0.2) (layer "B.Cu") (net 15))
 (segment (start 104.526 107.486) (end 104.526 114.45105) (width 0.2) (layer "B.Cu") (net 15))
 (segment (start 97.191 95.011) (end 96.04 93.86) (width 0.2) (layer "B.Cu") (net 15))
 (segment (start 102.96395 115.101) (end 97.191 109.32805) (width 0.2) (layer "B.Cu") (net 15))
 (segment (start 104.526 114.45105) (end 103.87605 115.101) (width 0.2) (layer "B.Cu") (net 15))
 (segment (start 121.2 88.6) (end 104.521 105.279) (width 0.2) (layer "F.Cu") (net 26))
 (segment (start 94.781 105.279) (end 93.5 106.56) (width 0.2) (layer "F.Cu") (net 26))
 (segment (start 104.521 105.279) (end 94.781 105.279) (width 0.2) (layer "F.Cu") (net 26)))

